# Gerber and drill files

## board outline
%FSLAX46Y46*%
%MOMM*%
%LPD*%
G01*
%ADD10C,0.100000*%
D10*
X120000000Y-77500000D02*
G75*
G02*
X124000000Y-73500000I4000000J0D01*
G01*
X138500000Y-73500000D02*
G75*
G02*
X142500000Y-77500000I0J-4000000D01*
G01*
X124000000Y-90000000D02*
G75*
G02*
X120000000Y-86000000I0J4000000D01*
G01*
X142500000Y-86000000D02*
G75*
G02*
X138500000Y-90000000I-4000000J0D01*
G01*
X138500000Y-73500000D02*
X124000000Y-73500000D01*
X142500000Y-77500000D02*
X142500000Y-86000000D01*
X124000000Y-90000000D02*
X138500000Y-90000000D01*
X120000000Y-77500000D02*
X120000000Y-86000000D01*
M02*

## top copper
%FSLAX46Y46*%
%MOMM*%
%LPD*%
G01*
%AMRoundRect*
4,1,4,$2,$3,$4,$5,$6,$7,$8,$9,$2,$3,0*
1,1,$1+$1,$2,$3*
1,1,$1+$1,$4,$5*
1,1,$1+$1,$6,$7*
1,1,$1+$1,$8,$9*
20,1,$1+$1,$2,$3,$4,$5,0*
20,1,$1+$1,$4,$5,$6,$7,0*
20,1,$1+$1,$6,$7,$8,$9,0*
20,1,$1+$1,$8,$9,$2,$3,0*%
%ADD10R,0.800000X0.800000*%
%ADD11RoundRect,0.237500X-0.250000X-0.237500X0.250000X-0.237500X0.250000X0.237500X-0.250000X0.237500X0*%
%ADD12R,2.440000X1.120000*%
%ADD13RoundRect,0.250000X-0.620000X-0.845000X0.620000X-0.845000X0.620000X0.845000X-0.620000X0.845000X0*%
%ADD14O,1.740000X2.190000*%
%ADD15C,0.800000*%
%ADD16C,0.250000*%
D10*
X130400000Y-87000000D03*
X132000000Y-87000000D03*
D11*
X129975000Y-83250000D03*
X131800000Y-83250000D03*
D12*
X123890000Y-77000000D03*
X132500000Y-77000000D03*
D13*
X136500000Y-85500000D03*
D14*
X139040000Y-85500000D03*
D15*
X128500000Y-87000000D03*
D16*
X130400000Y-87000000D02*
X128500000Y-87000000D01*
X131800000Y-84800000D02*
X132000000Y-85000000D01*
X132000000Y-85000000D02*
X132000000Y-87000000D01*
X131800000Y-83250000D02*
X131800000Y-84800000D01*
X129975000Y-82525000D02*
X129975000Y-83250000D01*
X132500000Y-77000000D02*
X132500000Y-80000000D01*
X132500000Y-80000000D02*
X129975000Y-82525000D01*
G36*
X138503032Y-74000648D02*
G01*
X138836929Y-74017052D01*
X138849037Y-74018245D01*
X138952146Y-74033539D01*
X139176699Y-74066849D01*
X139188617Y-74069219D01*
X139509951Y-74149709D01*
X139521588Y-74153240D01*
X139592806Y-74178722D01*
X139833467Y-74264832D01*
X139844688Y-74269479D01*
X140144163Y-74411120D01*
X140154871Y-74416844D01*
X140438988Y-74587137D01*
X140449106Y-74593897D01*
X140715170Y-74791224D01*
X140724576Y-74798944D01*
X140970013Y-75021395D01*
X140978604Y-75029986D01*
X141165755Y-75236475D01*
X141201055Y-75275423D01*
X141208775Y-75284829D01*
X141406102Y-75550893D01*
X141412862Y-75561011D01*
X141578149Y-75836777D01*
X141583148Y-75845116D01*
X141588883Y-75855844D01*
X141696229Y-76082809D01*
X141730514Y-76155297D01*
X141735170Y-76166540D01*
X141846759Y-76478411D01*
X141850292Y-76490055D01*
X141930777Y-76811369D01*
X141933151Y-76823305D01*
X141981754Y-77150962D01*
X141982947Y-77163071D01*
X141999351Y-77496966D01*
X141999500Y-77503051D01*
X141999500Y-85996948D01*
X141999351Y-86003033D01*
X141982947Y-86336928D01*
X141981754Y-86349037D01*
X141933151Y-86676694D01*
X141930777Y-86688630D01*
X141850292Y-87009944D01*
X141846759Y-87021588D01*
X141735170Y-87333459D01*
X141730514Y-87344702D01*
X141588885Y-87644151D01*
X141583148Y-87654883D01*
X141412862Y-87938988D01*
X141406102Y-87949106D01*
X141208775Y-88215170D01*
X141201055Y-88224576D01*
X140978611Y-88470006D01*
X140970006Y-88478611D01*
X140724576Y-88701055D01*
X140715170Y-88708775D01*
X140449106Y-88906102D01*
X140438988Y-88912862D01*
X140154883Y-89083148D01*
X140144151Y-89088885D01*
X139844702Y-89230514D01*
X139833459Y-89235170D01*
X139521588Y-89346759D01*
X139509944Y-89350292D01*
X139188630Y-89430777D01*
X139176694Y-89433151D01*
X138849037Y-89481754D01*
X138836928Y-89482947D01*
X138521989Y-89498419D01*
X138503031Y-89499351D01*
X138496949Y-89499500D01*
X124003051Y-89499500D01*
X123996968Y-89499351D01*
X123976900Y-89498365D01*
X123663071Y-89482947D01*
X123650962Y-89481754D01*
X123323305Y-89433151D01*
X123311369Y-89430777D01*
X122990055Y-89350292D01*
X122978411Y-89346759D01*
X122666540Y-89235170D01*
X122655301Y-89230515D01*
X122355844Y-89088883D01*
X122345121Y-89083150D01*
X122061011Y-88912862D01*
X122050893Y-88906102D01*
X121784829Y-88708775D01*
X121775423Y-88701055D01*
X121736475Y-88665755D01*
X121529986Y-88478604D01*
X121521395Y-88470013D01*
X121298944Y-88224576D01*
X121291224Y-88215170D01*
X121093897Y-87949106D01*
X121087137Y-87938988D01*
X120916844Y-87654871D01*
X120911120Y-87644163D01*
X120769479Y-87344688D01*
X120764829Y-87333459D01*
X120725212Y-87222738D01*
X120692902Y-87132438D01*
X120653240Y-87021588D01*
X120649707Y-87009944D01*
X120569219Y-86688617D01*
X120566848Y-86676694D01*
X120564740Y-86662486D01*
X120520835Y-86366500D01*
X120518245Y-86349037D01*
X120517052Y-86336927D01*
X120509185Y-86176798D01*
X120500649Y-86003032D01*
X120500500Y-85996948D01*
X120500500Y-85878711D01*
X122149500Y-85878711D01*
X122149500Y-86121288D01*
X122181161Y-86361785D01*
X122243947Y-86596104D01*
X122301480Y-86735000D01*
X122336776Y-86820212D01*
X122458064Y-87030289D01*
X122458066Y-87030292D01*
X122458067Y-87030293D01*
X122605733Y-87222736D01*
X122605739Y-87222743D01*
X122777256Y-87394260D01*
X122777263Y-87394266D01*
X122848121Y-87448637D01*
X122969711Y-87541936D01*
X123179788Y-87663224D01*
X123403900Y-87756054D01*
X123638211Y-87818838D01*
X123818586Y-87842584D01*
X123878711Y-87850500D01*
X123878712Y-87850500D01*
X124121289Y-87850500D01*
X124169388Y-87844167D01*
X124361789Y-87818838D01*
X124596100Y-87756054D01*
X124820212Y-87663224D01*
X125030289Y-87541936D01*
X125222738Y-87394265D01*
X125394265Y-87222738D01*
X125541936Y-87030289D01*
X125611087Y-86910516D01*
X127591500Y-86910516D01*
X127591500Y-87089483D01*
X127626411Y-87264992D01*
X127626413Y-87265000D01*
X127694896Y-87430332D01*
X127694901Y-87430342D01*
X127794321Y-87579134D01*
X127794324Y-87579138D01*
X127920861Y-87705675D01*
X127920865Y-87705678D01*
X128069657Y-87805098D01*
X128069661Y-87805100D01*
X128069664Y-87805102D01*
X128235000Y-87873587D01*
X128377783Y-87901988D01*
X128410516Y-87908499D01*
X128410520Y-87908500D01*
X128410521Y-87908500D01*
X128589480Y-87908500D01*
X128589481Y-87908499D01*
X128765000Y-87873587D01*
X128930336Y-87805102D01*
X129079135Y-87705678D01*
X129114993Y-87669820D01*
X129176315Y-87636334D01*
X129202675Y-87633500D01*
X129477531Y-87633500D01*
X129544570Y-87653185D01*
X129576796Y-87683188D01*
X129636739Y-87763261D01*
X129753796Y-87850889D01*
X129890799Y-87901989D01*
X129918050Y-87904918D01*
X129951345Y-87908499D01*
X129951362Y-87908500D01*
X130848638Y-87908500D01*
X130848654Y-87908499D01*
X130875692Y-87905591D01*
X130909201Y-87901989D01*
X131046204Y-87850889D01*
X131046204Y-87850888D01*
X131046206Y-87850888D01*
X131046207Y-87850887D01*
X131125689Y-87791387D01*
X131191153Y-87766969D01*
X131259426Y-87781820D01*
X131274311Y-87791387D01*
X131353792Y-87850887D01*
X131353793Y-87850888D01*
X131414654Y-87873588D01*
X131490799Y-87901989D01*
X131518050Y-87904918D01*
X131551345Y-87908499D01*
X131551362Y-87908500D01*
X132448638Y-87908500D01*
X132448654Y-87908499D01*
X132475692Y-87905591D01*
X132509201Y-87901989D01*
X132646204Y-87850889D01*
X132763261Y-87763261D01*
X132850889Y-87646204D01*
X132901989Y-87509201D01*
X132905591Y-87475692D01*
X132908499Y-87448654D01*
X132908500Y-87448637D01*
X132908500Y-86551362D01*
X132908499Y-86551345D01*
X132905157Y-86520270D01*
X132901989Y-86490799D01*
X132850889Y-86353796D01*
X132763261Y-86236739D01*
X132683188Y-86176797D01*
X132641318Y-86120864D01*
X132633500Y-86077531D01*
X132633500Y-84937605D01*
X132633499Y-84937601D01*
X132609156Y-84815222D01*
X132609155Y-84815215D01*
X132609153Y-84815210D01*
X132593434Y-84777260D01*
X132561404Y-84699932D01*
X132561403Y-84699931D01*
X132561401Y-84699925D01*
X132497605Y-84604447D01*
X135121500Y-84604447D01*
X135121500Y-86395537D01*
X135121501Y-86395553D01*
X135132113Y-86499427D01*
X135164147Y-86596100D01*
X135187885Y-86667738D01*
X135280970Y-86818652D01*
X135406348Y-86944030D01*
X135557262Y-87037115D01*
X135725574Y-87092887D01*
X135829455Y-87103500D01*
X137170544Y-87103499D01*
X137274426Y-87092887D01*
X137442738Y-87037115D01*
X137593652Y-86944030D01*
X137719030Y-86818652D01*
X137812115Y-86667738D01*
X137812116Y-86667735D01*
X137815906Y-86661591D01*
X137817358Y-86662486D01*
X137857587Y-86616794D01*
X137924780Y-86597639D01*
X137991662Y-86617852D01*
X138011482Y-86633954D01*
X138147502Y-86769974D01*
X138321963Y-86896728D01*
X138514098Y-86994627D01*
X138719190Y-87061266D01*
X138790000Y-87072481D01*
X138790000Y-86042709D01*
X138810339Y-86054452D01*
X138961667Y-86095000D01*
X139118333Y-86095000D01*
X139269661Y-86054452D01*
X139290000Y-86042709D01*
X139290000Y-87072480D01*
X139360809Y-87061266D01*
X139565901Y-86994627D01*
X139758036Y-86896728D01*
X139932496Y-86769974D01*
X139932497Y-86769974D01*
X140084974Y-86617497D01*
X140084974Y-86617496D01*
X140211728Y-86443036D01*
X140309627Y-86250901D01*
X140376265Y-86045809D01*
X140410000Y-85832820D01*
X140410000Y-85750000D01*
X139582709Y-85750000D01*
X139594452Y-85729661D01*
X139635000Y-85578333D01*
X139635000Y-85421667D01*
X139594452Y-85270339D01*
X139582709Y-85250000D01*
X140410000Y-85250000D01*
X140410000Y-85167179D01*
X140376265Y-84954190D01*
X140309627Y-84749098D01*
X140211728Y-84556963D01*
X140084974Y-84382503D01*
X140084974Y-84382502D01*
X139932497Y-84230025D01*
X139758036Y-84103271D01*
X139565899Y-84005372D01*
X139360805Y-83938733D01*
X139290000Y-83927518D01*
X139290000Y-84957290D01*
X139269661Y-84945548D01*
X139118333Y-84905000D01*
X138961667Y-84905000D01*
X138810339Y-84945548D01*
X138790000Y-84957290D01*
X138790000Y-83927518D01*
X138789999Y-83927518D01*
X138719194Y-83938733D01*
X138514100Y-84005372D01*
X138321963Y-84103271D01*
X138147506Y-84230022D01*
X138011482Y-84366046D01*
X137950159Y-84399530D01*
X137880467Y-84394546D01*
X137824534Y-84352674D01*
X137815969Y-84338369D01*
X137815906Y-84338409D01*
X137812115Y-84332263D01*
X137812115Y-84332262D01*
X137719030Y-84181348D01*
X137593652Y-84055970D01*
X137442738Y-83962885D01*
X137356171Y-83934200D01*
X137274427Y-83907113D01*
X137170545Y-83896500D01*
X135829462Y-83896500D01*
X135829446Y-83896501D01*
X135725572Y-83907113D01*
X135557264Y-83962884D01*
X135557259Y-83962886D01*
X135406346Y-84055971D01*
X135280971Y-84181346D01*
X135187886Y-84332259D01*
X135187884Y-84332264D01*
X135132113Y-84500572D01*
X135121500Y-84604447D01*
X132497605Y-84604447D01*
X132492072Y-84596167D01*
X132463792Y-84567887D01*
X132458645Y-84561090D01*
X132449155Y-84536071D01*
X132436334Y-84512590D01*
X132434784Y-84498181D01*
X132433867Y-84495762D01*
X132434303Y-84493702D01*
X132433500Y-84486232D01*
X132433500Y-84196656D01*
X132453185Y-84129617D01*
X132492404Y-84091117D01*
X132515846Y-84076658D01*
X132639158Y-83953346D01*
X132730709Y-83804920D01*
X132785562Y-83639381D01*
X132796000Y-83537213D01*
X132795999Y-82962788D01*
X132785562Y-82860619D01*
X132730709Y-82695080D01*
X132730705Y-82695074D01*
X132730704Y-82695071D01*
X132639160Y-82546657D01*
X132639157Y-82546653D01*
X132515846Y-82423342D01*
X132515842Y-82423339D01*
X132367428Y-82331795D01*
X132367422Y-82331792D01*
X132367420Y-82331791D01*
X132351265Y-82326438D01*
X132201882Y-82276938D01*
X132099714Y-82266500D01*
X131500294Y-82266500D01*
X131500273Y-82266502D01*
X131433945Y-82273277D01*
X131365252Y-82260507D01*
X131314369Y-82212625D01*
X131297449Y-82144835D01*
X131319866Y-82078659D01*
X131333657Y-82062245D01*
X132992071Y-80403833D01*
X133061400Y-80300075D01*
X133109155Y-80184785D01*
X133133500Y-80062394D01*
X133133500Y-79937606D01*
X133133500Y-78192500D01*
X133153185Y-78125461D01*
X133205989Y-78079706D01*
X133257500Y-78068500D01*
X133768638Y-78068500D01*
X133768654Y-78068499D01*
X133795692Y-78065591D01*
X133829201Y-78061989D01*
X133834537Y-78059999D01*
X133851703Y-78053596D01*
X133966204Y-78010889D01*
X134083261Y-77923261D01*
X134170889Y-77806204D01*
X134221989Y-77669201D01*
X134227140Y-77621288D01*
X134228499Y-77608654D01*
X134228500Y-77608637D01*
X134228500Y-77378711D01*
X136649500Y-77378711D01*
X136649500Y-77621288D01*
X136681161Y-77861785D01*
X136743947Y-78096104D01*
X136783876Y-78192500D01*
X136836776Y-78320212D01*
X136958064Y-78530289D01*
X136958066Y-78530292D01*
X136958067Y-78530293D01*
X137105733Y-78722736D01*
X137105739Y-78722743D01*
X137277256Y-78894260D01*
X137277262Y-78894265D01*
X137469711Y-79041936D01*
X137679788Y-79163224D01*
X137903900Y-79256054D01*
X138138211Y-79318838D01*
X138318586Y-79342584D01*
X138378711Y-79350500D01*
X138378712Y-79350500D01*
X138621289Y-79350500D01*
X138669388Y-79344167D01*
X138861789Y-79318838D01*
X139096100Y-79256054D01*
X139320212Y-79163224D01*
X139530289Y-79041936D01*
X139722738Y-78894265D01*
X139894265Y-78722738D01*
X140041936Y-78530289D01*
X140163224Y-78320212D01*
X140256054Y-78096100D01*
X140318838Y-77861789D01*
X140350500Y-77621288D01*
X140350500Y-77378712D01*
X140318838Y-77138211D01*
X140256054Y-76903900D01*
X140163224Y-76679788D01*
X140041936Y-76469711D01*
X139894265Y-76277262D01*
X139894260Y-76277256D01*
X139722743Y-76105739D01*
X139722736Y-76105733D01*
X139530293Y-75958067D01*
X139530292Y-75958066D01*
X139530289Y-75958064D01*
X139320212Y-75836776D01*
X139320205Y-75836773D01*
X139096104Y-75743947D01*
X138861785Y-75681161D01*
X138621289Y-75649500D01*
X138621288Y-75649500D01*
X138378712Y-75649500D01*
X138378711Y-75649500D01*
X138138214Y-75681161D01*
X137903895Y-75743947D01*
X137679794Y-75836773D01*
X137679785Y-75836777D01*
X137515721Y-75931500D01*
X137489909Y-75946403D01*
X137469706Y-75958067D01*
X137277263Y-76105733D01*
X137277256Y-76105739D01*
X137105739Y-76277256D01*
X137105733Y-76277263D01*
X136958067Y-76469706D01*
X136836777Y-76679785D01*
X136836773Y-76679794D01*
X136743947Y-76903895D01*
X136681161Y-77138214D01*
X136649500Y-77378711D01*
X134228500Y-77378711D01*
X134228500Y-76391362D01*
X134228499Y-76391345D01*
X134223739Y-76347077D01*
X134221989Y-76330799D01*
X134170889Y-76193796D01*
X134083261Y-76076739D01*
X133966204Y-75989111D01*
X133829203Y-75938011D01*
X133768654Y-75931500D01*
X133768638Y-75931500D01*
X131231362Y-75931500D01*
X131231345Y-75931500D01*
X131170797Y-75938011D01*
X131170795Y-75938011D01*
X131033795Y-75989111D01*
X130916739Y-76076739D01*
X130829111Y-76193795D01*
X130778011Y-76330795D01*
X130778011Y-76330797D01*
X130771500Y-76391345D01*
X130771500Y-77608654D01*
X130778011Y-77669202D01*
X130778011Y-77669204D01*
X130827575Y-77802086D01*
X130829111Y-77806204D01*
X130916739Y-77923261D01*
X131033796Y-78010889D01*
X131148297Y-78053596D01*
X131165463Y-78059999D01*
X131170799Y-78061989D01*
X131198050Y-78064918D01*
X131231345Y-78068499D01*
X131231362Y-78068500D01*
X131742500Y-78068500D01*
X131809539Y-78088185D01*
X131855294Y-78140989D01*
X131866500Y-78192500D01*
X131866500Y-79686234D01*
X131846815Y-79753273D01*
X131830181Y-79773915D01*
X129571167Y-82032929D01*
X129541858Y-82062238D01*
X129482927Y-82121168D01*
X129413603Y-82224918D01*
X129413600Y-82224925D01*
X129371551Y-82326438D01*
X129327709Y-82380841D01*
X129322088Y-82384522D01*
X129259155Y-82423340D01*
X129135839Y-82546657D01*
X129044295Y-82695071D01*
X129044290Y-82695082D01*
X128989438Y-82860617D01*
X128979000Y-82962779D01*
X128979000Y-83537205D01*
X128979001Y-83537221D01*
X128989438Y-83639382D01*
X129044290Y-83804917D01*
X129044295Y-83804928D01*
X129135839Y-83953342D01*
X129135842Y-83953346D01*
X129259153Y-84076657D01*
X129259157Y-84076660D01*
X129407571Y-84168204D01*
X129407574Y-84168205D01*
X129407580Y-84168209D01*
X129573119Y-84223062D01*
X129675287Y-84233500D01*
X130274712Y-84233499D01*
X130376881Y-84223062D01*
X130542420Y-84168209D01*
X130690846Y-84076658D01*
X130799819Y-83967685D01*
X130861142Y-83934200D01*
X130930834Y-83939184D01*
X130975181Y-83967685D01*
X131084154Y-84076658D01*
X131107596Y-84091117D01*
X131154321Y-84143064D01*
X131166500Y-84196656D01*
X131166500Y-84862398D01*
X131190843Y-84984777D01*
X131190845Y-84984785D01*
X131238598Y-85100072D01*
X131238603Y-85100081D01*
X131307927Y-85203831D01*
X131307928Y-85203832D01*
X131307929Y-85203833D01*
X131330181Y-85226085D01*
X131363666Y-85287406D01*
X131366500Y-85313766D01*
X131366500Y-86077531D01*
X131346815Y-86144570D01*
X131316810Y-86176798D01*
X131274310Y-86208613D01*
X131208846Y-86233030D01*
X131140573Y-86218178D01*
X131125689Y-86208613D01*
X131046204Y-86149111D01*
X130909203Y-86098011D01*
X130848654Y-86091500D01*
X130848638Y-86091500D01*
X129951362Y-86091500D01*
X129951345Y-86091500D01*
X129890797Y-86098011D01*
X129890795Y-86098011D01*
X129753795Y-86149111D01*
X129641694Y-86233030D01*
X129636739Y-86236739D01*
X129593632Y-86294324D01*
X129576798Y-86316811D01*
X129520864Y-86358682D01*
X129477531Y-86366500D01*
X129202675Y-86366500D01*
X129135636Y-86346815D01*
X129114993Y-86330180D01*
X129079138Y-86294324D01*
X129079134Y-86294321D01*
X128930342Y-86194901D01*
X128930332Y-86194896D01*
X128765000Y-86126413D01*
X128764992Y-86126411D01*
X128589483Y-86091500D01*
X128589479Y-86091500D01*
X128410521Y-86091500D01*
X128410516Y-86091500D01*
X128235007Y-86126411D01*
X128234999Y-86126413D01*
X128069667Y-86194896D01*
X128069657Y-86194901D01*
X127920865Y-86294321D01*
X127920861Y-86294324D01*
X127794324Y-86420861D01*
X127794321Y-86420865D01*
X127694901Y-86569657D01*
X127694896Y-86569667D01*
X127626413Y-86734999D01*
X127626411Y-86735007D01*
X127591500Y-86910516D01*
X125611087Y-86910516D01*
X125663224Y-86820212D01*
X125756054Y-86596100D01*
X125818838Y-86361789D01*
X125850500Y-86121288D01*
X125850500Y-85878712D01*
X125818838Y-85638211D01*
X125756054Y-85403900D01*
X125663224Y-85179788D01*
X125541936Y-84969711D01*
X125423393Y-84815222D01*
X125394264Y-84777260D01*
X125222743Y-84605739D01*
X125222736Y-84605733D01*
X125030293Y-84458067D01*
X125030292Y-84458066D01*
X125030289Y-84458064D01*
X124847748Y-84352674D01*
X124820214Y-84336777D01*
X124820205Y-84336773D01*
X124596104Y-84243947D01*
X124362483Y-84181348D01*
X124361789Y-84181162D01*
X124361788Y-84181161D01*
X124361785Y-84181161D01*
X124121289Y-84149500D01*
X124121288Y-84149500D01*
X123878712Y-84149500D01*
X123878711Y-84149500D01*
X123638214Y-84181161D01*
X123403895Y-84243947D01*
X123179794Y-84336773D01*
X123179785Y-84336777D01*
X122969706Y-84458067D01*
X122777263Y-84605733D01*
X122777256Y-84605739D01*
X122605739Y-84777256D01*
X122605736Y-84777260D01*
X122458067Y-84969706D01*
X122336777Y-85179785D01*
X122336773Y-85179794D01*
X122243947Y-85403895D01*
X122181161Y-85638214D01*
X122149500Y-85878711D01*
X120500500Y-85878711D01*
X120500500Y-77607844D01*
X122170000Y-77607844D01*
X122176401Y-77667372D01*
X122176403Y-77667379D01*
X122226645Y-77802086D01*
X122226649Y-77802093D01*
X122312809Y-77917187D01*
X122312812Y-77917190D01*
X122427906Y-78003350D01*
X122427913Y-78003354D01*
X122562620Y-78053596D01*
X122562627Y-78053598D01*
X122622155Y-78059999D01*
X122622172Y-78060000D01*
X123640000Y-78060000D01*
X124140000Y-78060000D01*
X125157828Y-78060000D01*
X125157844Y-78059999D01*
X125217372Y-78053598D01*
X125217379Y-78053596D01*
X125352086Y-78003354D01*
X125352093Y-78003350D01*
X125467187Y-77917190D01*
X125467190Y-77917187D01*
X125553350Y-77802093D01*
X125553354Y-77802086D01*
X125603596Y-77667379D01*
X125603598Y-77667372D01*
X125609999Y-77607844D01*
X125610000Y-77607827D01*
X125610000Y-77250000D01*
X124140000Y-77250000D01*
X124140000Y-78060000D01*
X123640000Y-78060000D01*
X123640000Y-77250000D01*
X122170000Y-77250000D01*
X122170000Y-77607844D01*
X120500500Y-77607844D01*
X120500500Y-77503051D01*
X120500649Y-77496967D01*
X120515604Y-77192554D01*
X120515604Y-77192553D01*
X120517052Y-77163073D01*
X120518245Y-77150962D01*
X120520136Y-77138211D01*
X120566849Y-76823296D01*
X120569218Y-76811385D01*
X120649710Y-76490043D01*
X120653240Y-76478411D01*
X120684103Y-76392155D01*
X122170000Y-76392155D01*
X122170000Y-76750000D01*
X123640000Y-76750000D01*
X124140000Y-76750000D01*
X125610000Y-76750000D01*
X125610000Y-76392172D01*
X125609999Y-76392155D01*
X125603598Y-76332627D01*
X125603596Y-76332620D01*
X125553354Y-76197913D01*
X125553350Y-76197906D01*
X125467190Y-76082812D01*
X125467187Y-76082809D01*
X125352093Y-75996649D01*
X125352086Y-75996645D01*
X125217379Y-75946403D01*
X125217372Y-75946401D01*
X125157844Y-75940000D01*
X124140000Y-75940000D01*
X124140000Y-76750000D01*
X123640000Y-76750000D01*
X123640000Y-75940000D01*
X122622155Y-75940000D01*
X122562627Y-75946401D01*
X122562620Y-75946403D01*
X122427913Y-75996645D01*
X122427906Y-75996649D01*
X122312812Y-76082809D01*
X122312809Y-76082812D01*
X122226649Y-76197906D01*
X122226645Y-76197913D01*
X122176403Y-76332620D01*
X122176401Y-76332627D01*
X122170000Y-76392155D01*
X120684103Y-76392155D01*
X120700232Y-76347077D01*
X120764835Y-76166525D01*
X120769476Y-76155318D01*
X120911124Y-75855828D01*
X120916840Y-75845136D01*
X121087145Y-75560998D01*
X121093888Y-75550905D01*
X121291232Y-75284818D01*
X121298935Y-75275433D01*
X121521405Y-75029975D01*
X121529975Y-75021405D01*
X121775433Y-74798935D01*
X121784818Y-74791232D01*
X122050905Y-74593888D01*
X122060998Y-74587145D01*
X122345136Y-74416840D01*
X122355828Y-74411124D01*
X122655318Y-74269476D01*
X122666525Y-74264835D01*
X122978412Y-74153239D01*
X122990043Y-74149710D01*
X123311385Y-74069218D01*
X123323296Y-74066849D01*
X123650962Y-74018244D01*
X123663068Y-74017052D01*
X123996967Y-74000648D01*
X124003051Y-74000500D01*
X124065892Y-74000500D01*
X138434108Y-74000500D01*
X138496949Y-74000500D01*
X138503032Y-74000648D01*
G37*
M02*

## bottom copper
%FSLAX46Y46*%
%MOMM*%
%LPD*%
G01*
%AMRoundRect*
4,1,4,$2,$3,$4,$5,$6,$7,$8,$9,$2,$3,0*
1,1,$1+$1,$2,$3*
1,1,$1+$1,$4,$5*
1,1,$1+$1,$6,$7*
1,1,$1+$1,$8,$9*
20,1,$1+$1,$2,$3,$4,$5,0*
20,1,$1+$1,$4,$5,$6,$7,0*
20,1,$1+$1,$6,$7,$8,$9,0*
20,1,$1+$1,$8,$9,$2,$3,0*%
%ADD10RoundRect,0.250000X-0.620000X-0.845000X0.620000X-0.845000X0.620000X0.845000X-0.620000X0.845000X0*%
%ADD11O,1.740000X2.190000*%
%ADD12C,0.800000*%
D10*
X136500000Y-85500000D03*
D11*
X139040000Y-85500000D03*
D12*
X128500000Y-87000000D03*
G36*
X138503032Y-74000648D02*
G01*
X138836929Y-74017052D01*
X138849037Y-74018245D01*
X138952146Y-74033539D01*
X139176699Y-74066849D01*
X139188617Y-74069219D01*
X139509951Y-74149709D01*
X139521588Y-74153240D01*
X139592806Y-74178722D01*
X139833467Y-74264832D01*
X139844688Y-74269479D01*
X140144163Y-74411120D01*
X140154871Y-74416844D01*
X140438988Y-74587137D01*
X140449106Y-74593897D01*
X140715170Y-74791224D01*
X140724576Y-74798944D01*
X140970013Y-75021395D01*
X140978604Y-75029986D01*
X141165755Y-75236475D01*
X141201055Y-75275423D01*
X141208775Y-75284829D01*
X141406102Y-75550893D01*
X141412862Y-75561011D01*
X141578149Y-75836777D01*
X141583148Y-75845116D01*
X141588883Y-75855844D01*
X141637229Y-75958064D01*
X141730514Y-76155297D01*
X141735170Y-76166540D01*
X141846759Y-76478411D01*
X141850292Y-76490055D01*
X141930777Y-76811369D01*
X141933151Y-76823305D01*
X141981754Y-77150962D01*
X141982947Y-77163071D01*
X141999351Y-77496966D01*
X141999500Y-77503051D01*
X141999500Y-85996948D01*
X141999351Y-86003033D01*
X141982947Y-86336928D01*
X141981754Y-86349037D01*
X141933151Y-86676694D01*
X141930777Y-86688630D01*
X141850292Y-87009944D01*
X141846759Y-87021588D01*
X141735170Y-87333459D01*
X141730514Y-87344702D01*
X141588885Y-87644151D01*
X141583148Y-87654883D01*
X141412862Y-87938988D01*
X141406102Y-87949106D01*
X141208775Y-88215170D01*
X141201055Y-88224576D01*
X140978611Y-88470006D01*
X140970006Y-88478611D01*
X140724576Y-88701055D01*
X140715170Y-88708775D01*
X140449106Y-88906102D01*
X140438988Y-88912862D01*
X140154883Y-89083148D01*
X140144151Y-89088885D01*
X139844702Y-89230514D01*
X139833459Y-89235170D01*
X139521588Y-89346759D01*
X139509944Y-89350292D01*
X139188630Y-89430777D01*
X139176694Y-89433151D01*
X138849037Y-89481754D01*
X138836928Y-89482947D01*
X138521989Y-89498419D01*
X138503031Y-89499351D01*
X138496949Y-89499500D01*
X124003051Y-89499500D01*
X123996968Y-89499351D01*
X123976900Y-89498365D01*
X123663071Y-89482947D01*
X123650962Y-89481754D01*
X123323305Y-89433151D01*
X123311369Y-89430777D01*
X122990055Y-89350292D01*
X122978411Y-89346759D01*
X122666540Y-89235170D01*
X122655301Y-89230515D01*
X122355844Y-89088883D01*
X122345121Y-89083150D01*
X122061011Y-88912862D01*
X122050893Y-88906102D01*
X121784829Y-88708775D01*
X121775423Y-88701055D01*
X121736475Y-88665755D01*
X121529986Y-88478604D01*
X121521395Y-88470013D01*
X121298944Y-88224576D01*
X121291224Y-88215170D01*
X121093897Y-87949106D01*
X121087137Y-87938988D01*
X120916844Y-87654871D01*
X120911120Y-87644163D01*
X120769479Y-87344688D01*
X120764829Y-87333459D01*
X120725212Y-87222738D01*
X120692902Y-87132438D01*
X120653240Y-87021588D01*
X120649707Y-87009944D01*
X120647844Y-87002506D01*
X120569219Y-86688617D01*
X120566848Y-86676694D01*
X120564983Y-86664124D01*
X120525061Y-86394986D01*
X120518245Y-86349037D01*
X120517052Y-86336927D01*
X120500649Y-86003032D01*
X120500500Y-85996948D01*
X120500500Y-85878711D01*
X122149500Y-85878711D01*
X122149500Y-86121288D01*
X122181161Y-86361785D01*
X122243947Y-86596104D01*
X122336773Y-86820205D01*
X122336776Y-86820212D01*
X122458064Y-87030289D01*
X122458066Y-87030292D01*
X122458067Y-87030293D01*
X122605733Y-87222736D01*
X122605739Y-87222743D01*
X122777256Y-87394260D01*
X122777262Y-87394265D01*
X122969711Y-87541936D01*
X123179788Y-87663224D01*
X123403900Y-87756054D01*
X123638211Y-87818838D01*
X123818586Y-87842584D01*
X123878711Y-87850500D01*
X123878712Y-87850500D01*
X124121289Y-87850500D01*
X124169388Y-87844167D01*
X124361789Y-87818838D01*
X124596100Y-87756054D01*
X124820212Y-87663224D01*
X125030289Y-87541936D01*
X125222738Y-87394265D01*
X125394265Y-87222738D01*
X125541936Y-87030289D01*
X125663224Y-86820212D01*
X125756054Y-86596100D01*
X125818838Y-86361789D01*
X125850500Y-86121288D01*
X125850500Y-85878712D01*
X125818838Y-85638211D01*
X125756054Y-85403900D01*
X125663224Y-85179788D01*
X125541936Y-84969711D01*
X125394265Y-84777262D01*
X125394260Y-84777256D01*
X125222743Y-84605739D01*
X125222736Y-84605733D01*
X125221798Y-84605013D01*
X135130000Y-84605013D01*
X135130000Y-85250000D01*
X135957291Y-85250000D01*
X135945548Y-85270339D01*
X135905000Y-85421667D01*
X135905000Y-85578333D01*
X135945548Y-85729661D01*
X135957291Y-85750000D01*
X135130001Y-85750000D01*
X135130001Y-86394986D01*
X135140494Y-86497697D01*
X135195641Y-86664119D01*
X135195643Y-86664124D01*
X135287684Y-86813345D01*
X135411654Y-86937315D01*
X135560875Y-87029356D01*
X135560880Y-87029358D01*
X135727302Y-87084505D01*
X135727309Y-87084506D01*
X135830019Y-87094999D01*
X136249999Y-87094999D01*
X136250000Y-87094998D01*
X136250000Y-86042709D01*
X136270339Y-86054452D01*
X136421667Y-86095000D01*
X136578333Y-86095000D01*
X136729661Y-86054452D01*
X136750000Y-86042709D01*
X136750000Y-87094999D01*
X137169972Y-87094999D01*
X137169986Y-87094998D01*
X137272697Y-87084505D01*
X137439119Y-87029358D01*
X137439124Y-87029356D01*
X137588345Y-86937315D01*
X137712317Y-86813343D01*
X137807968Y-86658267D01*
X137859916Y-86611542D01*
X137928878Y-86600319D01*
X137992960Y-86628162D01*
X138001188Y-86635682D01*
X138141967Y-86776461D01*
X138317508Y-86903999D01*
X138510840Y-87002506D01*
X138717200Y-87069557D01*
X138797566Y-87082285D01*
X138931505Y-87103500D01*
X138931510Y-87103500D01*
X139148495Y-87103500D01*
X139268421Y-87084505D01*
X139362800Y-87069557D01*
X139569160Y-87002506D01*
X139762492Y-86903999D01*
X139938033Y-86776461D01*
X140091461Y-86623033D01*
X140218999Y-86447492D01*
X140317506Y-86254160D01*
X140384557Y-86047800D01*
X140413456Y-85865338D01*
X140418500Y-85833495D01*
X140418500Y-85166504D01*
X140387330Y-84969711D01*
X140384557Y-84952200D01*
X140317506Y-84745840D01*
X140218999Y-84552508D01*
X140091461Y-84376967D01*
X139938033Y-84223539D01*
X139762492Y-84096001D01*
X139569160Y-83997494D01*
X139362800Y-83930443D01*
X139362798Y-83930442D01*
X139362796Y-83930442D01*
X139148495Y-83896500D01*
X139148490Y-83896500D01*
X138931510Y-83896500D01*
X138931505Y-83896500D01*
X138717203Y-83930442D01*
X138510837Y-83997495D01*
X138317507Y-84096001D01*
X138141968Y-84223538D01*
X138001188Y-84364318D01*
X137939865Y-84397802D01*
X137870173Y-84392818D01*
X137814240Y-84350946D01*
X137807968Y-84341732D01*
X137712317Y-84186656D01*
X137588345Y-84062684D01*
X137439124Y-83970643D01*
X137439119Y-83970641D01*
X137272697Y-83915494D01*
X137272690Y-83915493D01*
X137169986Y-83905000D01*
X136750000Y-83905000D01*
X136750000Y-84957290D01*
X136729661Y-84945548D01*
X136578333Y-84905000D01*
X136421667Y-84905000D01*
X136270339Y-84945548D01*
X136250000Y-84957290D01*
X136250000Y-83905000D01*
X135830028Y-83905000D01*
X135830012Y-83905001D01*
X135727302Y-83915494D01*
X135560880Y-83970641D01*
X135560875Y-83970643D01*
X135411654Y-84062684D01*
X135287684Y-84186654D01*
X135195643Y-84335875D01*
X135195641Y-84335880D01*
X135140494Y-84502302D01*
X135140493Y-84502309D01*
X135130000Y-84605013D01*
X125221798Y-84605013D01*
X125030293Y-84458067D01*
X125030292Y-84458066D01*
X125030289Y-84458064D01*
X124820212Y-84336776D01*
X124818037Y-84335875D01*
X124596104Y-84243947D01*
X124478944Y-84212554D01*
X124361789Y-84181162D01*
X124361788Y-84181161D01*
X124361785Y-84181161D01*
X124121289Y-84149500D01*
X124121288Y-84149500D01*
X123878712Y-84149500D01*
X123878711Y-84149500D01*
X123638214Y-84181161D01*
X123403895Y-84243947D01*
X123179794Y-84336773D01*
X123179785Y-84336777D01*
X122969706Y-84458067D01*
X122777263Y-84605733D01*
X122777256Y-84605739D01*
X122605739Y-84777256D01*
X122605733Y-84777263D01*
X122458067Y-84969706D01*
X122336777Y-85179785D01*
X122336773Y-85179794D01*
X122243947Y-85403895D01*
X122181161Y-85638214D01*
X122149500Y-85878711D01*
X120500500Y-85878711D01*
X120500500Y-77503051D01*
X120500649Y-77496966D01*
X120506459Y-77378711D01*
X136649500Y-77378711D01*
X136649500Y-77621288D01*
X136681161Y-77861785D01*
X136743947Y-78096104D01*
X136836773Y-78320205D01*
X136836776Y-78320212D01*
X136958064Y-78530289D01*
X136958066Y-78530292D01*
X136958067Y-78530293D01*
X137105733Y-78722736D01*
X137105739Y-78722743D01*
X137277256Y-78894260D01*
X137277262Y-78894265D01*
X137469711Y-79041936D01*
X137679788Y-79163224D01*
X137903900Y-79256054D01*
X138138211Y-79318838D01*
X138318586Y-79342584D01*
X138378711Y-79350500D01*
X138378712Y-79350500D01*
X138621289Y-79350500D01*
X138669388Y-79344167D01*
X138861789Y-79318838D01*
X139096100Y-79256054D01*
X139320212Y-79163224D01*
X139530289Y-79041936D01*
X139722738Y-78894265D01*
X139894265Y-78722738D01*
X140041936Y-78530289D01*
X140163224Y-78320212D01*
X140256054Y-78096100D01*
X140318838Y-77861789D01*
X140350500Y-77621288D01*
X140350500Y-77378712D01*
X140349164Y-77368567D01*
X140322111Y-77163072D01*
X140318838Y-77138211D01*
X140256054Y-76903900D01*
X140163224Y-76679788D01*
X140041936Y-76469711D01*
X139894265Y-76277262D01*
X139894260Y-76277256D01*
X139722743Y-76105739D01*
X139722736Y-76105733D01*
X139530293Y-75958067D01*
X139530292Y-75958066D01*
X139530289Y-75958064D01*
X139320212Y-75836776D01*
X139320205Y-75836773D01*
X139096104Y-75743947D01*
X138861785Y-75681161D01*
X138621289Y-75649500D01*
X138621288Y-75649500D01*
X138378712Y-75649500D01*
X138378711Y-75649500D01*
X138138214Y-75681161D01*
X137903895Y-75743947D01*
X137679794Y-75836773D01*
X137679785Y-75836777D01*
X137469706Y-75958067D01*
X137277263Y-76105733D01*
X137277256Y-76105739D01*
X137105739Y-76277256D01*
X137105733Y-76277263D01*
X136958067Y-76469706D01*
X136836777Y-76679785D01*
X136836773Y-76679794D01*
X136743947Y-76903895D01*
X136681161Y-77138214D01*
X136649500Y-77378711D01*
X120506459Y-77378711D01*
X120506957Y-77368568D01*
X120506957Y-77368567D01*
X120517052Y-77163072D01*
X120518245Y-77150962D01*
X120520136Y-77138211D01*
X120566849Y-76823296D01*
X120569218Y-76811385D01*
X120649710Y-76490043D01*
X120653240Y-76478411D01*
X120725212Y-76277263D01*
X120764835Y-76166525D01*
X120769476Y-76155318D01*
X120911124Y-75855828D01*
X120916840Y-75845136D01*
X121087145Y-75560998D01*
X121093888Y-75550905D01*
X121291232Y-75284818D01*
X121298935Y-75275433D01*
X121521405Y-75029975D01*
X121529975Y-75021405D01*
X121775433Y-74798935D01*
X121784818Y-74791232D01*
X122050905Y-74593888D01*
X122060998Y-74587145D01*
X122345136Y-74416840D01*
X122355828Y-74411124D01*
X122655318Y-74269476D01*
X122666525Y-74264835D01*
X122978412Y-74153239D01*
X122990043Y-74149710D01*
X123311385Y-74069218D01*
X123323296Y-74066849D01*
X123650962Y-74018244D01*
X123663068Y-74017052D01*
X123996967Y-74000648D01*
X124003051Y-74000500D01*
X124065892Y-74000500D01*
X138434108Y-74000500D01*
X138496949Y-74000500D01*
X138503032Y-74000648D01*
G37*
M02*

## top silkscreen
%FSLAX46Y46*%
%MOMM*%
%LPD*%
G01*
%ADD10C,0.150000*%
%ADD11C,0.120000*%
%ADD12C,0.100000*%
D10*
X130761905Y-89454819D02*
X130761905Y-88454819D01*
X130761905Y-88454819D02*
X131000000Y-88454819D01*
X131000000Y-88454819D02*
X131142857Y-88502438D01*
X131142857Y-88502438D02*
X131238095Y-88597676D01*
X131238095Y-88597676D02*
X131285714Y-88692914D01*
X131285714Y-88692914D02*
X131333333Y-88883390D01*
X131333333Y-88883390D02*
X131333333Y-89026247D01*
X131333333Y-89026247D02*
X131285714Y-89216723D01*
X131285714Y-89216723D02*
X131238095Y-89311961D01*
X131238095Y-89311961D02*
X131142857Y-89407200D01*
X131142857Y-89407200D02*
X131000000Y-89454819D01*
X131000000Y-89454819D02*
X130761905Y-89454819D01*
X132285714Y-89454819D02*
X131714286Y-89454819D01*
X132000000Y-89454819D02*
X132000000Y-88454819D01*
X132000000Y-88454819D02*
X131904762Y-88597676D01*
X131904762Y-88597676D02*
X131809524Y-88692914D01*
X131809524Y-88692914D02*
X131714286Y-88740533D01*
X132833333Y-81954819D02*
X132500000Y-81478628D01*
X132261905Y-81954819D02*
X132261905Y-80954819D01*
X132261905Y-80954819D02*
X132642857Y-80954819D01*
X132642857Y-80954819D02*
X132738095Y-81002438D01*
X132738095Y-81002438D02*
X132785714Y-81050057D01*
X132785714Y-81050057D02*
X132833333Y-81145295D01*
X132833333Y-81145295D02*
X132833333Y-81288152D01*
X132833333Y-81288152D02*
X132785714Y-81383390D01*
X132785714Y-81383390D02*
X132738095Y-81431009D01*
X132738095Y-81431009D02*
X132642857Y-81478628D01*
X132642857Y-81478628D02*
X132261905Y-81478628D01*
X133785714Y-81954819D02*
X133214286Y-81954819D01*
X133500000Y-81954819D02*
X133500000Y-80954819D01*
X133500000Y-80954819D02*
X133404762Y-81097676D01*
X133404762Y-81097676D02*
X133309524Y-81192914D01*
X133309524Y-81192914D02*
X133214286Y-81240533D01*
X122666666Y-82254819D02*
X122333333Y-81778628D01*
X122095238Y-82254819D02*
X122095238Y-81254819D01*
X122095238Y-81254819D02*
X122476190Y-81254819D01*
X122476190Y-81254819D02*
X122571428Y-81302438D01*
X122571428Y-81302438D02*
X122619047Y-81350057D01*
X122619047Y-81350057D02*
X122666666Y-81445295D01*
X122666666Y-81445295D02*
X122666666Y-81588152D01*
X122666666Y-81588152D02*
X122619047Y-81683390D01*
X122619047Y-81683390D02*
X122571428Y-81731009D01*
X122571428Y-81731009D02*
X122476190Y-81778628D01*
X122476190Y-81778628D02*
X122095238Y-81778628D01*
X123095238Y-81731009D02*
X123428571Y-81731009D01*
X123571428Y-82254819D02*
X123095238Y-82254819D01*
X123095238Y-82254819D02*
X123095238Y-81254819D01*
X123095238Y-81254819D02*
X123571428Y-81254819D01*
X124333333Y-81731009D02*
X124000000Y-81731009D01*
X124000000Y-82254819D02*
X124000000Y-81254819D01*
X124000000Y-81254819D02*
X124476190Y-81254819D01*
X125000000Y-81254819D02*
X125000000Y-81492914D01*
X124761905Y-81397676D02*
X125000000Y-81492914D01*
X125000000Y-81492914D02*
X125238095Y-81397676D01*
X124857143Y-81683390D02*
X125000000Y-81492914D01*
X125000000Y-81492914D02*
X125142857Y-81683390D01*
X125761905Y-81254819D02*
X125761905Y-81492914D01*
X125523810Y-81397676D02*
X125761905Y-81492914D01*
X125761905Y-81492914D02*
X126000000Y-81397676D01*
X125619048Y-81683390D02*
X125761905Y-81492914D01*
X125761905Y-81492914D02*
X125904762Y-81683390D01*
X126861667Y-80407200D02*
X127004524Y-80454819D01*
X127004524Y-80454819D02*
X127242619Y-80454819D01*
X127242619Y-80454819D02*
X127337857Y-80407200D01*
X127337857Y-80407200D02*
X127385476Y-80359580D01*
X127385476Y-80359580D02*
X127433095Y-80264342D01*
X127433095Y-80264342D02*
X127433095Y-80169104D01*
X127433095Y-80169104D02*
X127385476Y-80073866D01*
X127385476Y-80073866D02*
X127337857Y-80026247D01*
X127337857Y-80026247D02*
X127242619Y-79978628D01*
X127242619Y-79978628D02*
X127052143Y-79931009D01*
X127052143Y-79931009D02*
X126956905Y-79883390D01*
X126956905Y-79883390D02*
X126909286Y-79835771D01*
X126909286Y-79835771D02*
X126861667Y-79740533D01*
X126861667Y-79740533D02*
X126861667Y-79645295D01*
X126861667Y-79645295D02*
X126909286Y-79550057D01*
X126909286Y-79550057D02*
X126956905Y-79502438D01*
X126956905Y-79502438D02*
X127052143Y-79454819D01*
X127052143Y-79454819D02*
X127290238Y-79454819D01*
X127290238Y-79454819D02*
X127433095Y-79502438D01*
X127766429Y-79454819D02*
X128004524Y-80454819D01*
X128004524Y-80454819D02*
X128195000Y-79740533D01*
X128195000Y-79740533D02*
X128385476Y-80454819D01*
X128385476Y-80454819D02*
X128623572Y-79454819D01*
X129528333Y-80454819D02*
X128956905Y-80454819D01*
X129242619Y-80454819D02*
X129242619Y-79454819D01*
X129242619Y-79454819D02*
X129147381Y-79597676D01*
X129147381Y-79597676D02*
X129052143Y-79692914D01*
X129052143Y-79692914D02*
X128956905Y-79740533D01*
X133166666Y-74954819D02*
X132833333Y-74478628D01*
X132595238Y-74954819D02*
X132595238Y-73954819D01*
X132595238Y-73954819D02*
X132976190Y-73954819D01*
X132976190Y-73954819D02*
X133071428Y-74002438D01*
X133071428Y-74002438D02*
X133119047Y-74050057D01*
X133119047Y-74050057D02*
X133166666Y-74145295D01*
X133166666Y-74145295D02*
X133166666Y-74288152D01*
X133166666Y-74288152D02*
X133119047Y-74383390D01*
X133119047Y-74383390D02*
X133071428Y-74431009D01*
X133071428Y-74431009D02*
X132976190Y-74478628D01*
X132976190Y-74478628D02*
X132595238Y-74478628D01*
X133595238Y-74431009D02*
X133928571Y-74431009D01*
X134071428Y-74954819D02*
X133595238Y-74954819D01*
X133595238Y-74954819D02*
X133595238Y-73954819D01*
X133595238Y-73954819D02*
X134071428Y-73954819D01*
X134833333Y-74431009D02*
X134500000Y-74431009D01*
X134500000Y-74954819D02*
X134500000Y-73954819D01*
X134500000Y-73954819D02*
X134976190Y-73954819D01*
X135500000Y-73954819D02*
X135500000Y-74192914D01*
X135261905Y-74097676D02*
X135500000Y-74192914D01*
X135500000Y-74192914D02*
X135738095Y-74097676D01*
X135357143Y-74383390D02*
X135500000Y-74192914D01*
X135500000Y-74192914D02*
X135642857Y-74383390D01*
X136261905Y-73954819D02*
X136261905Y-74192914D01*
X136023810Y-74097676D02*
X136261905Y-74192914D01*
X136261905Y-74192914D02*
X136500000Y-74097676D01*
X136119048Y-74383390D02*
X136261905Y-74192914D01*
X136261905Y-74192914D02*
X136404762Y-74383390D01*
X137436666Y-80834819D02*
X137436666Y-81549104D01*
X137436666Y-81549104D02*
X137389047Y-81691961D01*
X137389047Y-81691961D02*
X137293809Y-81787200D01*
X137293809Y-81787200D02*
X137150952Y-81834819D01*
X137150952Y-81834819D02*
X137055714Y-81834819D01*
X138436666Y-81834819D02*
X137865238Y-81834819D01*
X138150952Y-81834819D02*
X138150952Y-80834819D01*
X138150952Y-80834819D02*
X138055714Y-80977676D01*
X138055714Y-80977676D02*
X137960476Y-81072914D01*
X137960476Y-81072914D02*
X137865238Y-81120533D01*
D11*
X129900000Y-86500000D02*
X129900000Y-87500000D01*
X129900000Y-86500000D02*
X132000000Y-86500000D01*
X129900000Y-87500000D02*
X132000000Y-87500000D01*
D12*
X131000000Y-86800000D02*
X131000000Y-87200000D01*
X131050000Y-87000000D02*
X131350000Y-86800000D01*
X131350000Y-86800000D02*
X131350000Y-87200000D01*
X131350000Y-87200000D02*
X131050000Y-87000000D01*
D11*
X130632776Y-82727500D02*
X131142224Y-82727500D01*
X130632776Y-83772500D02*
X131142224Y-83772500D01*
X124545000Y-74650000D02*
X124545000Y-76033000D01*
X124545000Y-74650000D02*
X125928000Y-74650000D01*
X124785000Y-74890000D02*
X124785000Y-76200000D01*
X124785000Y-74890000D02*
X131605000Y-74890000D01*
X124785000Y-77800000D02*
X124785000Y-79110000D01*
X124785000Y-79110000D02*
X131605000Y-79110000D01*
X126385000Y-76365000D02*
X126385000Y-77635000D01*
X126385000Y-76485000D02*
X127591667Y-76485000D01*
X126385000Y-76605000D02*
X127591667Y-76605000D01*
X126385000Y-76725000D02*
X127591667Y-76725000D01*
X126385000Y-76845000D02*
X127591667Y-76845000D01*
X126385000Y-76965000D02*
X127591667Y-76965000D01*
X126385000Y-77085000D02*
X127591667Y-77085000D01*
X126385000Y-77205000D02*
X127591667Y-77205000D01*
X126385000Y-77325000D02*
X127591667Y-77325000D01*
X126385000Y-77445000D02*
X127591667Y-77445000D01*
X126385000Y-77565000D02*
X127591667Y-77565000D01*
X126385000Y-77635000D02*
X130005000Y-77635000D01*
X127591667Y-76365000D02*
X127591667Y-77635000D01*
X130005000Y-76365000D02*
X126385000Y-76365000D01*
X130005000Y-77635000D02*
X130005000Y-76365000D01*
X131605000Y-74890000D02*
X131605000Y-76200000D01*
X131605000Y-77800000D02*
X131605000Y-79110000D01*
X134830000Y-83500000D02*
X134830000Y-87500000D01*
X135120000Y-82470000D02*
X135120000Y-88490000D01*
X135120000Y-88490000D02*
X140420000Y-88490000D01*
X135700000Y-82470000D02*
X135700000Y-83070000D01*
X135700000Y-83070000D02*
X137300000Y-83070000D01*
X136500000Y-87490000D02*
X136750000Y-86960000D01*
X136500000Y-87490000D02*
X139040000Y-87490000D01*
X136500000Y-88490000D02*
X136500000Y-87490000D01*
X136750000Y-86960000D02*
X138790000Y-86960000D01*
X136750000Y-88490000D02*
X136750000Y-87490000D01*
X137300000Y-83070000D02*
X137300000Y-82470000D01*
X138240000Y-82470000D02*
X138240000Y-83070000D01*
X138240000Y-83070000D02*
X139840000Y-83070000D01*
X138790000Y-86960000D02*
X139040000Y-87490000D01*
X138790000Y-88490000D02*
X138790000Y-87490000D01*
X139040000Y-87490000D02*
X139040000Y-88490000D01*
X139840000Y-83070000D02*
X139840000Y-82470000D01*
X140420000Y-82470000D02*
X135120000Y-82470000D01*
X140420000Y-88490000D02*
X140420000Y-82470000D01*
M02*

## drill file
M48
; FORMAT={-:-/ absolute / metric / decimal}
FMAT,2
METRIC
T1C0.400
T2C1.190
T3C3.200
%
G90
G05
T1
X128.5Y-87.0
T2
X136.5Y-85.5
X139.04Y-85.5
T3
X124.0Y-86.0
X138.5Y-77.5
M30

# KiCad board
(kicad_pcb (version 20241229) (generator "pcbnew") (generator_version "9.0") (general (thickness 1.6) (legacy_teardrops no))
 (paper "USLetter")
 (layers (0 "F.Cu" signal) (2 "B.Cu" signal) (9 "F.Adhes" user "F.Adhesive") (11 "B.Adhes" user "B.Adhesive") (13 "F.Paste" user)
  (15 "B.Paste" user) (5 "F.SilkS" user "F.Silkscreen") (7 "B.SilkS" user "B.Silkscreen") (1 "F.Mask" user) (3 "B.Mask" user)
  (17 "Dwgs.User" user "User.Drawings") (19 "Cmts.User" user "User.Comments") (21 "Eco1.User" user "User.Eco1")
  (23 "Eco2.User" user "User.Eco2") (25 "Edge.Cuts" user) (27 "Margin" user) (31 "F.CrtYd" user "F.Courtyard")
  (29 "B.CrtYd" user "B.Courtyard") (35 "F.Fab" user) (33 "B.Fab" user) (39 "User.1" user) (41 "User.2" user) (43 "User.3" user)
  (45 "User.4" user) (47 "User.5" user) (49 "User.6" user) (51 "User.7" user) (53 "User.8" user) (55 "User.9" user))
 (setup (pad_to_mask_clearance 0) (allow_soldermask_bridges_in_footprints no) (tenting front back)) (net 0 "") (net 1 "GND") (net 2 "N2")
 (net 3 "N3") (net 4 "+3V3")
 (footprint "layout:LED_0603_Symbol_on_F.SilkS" (layer "F.Cu") (at 131.2 87)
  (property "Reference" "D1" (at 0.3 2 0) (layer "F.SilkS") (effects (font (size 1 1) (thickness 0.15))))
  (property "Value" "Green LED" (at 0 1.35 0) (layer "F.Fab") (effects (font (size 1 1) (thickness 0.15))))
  (fp_line (start -1.3 -0.5) (end -1.3 0.5) (stroke (width 0.12) (type solid)) (layer "F.SilkS"))
  (fp_line (start -1.3 -0.5) (end 0.8 -0.5) (stroke (width 0.12) (type solid)) (layer "F.SilkS"))
  (fp_line (start -1.3 0.5) (end 0.8 0.5) (stroke (width 0.12) (type solid)) (layer "F.SilkS"))
  (fp_line (start -0.2 -0.2) (end -0.2 0.2) (stroke (width 0.1) (type solid)) (layer "F.SilkS"))
  (fp_line (start -0.15 0) (end 0.15 -0.2) (stroke (width 0.1) (type solid)) (layer "F.SilkS"))
  (fp_line (start 0.15 -0.2) (end 0.15 0.2) (stroke (width 0.1) (type solid)) (layer "F.SilkS"))
  (fp_line (start 0.15 0.2) (end -0.15 0) (stroke (width 0.1) (type solid)) (layer "F.SilkS"))
  (pad "1" smd rect (at -0.8 0 180) (size 0.8 0.8) (layers "F.Cu" "F.Mask" "F.Paste") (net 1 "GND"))
  (pad "2" smd rect (at 0.8 0 180) (size 0.8 0.8) (layers "F.Cu" "F.Mask" "F.Paste") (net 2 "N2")))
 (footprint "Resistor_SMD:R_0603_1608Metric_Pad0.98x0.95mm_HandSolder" (layer "F.Cu") (at 130.8875 83.25)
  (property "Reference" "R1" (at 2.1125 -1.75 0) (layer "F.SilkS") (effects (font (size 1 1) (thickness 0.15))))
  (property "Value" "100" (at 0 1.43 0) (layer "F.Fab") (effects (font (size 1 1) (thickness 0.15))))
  (fp_line (start -0.254724 -0.5225) (end 0.254724 -0.5225) (stroke (width 0.12) (type solid)) (layer "F.SilkS"))
  (fp_line (start -0.254724 0.5225) (end 0.254724 0.5225) (stroke (width 0.12) (type solid)) (layer "F.SilkS"))
  (pad "1" smd roundrect (at -0.9125 0) (size 0.975 0.95) (layers "F.Cu" "F.Mask" "F.Paste") (roundrect_rratio 0.25) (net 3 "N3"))
  (pad "2" smd roundrect (at 0.9125 0) (size 0.975 0.95) (layers "F.Cu" "F.Mask" "F.Paste") (roundrect_rratio 0.25) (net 2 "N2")))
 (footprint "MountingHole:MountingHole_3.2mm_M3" (layer "F.Cu") (at 124 86)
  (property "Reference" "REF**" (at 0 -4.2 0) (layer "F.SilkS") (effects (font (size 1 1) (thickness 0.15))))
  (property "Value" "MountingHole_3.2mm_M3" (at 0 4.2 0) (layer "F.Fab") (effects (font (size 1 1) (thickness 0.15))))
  (pad "" np_thru_hole circle (at 0 0) (size 3.2 3.2) (drill 3.2) (layers "*.Cu" "*.Mask")))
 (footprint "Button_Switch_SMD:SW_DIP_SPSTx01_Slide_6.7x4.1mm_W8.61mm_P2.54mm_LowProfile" (layer "F.Cu") (at 128.195 77)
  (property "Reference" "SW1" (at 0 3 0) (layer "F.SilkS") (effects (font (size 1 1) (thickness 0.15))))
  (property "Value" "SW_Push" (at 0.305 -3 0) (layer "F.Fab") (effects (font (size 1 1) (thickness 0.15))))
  (fp_line (start -3.65 -2.35) (end -3.65 -0.967) (stroke (width 0.12) (type solid)) (layer "F.SilkS"))
  (fp_line (start -3.65 -2.35) (end -2.267 -2.35) (stroke (width 0.12) (type solid)) (layer "F.SilkS"))
  (fp_line (start -3.41 -2.11) (end -3.41 -0.8) (stroke (width 0.12) (type solid)) (layer "F.SilkS"))
  (fp_line (start -3.41 -2.11) (end 3.41 -2.11) (stroke (width 0.12) (type solid)) (layer "F.SilkS"))
  (fp_line (start -3.41 0.8) (end -3.41 2.11) (stroke (width 0.12) (type solid)) (layer "F.SilkS"))
  (fp_line (start -3.41 2.11) (end 3.41 2.11) (stroke (width 0.12) (type solid)) (layer "F.SilkS"))
  (fp_line (start -1.81 -0.635) (end -1.81 0.635) (stroke (width 0.12) (type solid)) (layer "F.SilkS"))
  (fp_line (start -1.81 -0.515) (end -0.603333 -0.515) (stroke (width 0.12) (type solid)) (layer "F.SilkS"))
  (fp_line (start -1.81 -0.395) (end -0.603333 -0.395) (stroke (width 0.12) (type solid)) (layer "F.SilkS"))
  (fp_line (start -1.81 -0.275) (end -0.603333 -0.275) (stroke (width 0.12) (type solid)) (layer "F.SilkS"))
  (fp_line (start -1.81 -0.155) (end -0.603333 -0.155) (stroke (width 0.12) (type solid)) (layer "F.SilkS"))
  (fp_line (start -1.81 -0.035) (end -0.603333 -0.035) (stroke (width 0.12) (type solid)) (layer "F.SilkS"))
  (fp_line (start -1.81 0.085) (end -0.603333 0.085) (stroke (width 0.12) (type solid)) (layer "F.SilkS"))
  (fp_line (start -1.81 0.205) (end -0.603333 0.205) (stroke (width 0.12) (type solid)) (layer "F.SilkS"))
  (fp_line (start -1.81 0.325) (end -0.603333 0.325) (stroke (width 0.12) (type solid)) (layer "F.SilkS"))
  (fp_line (start -1.81 0.445) (end -0.603333 0.445) (stroke (width 0.12) (type solid)) (layer "F.SilkS"))
  (fp_line (start -1.81 0.565) (end -0.603333 0.565) (stroke (width 0.12) (type solid)) (layer "F.SilkS"))
  (fp_line (start -1.81 0.635) (end 1.81 0.635) (stroke (width 0.12) (type solid)) (layer "F.SilkS"))
  (fp_line (start -0.603333 -0.635) (end -0.603333 0.635) (stroke (width 0.12) (type solid)) (layer "F.SilkS"))
  (fp_line (start 1.81 -0.635) (end -1.81 -0.635) (stroke (width 0.12) (type solid)) (layer "F.SilkS"))
  (fp_line (start 1.81 0.635) (end 1.81 -0.635) (stroke (width 0.12) (type solid)) (layer "F.SilkS"))
  (fp_line (start 3.41 -2.11) (end 3.41 -0.8) (stroke (width 0.12) (type solid)) (layer "F.SilkS"))
  (fp_line (start 3.41 0.8) (end 3.41 2.11) (stroke (width 0.12) (type solid)) (layer "F.SilkS"))
  (pad "1" smd rect (at -4.305 0) (size 2.44 1.12) (layers "F.Cu" "F.Mask" "F.Paste") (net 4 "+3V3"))
  (pad "2" smd rect (at 4.305 0) (size 2.44 1.12) (layers "F.Cu" "F.Mask" "F.Paste") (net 3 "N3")))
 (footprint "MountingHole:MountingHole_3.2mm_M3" (layer "F.Cu") (at 138.5 77.5)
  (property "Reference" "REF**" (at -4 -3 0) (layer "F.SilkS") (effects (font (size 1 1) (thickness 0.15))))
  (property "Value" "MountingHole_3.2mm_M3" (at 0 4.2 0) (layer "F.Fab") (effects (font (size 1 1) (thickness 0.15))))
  (pad "" np_thru_hole circle (at 0 0) (size 3.2 3.2) (drill 3.2) (layers "*.Cu" "*.Mask")))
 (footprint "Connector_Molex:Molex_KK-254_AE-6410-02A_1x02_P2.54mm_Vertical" (layer "F.Cu") (at 136.5 85.5)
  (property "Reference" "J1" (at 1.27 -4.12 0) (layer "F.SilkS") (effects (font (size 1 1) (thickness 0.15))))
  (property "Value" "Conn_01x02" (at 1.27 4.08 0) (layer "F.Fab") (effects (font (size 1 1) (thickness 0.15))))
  (fp_line (start -1.67 -2) (end -1.67 2) (stroke (width 0.12) (type solid)) (layer "F.SilkS"))
  (fp_line (start -1.38 -3.03) (end -1.38 2.99) (stroke (width 0.12) (type solid)) (layer "F.SilkS"))
  (fp_line (start -1.38 2.99) (end 3.92 2.99) (stroke (width 0.12) (type solid)) (layer "F.SilkS"))
  (fp_line (start -0.8 -3.03) (end -0.8 -2.43) (stroke (width 0.12) (type solid)) (layer "F.SilkS"))
  (fp_line (start -0.8 -2.43) (end 0.8 -2.43) (stroke (width 0.12) (type solid)) (layer "F.SilkS"))
  (fp_line (start 0 1.99) (end 0.25 1.46) (stroke (width 0.12) (type solid)) (layer "F.SilkS"))
  (fp_line (start 0 1.99) (end 2.54 1.99) (stroke (width 0.12) (type solid)) (layer "F.SilkS"))
  (fp_line (start 0 2.99) (end 0 1.99) (stroke (width 0.12) (type solid)) (layer "F.SilkS"))
  (fp_line (start 0.25 1.46) (end 2.29 1.46) (stroke (width 0.12) (type solid)) (layer "F.SilkS"))
  (fp_line (start 0.25 2.99) (end 0.25 1.99) (stroke (width 0.12) (type solid)) (layer "F.SilkS"))
  (fp_line (start 0.8 -2.43) (end 0.8 -3.03) (stroke (width 0.12) (type solid)) (layer "F.SilkS"))
  (fp_line (start 1.74 -3.03) (end 1.74 -2.43) (stroke (width 0.12) (type solid)) (layer "F.SilkS"))
  (fp_line (start 1.74 -2.43) (end 3.34 -2.43) (stroke (width 0.12) (type solid)) (layer "F.SilkS"))
  (fp_line (start 2.29 1.46) (end 2.54 1.99) (stroke (width 0.12) (type solid)) (layer "F.SilkS"))
  (fp_line (start 2.29 2.99) (end 2.29 1.99) (stroke (width 0.12) (type solid)) (layer "F.SilkS"))
  (fp_line (start 2.54 1.99) (end 2.54 2.99) (stroke (width 0.12) (type solid)) (layer "F.SilkS"))
  (fp_line (start 3.34 -2.43) (end 3.34 -3.03) (stroke (width 0.12) (type solid)) (layer "F.SilkS"))
  (fp_line (start 3.92 -3.03) (end -1.38 -3.03) (stroke (width 0.12) (type solid)) (layer "F.SilkS"))
  (fp_line (start 3.92 2.99) (end 3.92 -3.03) (stroke (width 0.12) (type solid)) (layer "F.SilkS"))
  (pad "1" thru_hole roundrect (at 0 0) (size 1.74 2.19) (drill 1.19) (layers "*.Cu" "*.Mask") (remove_unused_layers no)
   (roundrect_rratio 0.143678) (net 1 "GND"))
  (pad "2" thru_hole oval (at 2.54 0) (size 1.74 2.19) (drill 1.19) (layers "*.Cu" "*.Mask") (remove_unused_layers no) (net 4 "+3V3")))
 (gr_arc (start 120 77.5) (mid 121.171573 74.671573) (end 124 73.5) (stroke (width 0.1) (type default)) (layer "Edge.Cuts"))
 (gr_arc (start 138.5 73.5) (mid 141.328427 74.671573) (end 142.5 77.5) (stroke (width 0.1) (type default)) (layer "Edge.Cuts"))
 (gr_arc (start 124 90) (mid 121.171573 88.828427) (end 120 86) (stroke (width 0.1) (type default)) (layer "Edge.Cuts"))
 (gr_arc (start 142.5 86) (mid 141.328427 88.828427) (end 138.5 90) (stroke (width 0.1) (type default)) (layer "Edge.Cuts"))
 (gr_line (start 138.5 73.5) (end 124 73.5) (stroke (width 0.1) (type default)) (layer "Edge.Cuts"))
 (gr_line (start 142.5 77.5) (end 142.5 86) (stroke (width 0.1) (type default)) (layer "Edge.Cuts"))
 (gr_line (start 124 90) (end 138.5 90) (stroke (width 0.1) (type default)) (layer "Edge.Cuts"))
 (gr_line (start 120 77.5) (end 120 86) (stroke (width 0.1) (type default)) (layer "Edge.Cuts"))
 (segment (start 130.4 87) (end 128.5 87) (width 0.25) (layer "F.Cu") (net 1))
 (via (at 128.5 87) (size 0.8) (drill 0.4) (layers "F.Cu" "B.Cu") (free yes) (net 1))
 (segment (start 131.8 84.8) (end 132 85) (width 0.25) (layer "F.Cu") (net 2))
 (segment (start 132 85) (end 132 87) (width 0.25) (layer "F.Cu") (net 2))
 (segment (start 131.8 83.25) (end 131.8 84.8) (width 0.25) (layer "F.Cu") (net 2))
 (segment (start 129.975 82.525) (end 129.975 83.25) (width 0.25) (layer "F.Cu") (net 3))
 (segment (start 132.5 77) (end 132.5 80) (width 0.25) (layer "F.Cu") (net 3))
 (segment (start 132.5 80) (end 129.975 82.525) (width 0.25) (layer "F.Cu") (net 3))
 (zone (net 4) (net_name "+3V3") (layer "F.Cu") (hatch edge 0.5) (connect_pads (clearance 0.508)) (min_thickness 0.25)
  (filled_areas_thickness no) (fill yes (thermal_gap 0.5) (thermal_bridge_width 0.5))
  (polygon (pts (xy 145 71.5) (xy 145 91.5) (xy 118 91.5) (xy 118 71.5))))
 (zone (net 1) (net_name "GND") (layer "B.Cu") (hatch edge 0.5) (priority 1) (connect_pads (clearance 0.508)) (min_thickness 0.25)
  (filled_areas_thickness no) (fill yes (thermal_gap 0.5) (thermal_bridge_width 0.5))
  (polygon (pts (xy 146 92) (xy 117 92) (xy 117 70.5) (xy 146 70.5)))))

